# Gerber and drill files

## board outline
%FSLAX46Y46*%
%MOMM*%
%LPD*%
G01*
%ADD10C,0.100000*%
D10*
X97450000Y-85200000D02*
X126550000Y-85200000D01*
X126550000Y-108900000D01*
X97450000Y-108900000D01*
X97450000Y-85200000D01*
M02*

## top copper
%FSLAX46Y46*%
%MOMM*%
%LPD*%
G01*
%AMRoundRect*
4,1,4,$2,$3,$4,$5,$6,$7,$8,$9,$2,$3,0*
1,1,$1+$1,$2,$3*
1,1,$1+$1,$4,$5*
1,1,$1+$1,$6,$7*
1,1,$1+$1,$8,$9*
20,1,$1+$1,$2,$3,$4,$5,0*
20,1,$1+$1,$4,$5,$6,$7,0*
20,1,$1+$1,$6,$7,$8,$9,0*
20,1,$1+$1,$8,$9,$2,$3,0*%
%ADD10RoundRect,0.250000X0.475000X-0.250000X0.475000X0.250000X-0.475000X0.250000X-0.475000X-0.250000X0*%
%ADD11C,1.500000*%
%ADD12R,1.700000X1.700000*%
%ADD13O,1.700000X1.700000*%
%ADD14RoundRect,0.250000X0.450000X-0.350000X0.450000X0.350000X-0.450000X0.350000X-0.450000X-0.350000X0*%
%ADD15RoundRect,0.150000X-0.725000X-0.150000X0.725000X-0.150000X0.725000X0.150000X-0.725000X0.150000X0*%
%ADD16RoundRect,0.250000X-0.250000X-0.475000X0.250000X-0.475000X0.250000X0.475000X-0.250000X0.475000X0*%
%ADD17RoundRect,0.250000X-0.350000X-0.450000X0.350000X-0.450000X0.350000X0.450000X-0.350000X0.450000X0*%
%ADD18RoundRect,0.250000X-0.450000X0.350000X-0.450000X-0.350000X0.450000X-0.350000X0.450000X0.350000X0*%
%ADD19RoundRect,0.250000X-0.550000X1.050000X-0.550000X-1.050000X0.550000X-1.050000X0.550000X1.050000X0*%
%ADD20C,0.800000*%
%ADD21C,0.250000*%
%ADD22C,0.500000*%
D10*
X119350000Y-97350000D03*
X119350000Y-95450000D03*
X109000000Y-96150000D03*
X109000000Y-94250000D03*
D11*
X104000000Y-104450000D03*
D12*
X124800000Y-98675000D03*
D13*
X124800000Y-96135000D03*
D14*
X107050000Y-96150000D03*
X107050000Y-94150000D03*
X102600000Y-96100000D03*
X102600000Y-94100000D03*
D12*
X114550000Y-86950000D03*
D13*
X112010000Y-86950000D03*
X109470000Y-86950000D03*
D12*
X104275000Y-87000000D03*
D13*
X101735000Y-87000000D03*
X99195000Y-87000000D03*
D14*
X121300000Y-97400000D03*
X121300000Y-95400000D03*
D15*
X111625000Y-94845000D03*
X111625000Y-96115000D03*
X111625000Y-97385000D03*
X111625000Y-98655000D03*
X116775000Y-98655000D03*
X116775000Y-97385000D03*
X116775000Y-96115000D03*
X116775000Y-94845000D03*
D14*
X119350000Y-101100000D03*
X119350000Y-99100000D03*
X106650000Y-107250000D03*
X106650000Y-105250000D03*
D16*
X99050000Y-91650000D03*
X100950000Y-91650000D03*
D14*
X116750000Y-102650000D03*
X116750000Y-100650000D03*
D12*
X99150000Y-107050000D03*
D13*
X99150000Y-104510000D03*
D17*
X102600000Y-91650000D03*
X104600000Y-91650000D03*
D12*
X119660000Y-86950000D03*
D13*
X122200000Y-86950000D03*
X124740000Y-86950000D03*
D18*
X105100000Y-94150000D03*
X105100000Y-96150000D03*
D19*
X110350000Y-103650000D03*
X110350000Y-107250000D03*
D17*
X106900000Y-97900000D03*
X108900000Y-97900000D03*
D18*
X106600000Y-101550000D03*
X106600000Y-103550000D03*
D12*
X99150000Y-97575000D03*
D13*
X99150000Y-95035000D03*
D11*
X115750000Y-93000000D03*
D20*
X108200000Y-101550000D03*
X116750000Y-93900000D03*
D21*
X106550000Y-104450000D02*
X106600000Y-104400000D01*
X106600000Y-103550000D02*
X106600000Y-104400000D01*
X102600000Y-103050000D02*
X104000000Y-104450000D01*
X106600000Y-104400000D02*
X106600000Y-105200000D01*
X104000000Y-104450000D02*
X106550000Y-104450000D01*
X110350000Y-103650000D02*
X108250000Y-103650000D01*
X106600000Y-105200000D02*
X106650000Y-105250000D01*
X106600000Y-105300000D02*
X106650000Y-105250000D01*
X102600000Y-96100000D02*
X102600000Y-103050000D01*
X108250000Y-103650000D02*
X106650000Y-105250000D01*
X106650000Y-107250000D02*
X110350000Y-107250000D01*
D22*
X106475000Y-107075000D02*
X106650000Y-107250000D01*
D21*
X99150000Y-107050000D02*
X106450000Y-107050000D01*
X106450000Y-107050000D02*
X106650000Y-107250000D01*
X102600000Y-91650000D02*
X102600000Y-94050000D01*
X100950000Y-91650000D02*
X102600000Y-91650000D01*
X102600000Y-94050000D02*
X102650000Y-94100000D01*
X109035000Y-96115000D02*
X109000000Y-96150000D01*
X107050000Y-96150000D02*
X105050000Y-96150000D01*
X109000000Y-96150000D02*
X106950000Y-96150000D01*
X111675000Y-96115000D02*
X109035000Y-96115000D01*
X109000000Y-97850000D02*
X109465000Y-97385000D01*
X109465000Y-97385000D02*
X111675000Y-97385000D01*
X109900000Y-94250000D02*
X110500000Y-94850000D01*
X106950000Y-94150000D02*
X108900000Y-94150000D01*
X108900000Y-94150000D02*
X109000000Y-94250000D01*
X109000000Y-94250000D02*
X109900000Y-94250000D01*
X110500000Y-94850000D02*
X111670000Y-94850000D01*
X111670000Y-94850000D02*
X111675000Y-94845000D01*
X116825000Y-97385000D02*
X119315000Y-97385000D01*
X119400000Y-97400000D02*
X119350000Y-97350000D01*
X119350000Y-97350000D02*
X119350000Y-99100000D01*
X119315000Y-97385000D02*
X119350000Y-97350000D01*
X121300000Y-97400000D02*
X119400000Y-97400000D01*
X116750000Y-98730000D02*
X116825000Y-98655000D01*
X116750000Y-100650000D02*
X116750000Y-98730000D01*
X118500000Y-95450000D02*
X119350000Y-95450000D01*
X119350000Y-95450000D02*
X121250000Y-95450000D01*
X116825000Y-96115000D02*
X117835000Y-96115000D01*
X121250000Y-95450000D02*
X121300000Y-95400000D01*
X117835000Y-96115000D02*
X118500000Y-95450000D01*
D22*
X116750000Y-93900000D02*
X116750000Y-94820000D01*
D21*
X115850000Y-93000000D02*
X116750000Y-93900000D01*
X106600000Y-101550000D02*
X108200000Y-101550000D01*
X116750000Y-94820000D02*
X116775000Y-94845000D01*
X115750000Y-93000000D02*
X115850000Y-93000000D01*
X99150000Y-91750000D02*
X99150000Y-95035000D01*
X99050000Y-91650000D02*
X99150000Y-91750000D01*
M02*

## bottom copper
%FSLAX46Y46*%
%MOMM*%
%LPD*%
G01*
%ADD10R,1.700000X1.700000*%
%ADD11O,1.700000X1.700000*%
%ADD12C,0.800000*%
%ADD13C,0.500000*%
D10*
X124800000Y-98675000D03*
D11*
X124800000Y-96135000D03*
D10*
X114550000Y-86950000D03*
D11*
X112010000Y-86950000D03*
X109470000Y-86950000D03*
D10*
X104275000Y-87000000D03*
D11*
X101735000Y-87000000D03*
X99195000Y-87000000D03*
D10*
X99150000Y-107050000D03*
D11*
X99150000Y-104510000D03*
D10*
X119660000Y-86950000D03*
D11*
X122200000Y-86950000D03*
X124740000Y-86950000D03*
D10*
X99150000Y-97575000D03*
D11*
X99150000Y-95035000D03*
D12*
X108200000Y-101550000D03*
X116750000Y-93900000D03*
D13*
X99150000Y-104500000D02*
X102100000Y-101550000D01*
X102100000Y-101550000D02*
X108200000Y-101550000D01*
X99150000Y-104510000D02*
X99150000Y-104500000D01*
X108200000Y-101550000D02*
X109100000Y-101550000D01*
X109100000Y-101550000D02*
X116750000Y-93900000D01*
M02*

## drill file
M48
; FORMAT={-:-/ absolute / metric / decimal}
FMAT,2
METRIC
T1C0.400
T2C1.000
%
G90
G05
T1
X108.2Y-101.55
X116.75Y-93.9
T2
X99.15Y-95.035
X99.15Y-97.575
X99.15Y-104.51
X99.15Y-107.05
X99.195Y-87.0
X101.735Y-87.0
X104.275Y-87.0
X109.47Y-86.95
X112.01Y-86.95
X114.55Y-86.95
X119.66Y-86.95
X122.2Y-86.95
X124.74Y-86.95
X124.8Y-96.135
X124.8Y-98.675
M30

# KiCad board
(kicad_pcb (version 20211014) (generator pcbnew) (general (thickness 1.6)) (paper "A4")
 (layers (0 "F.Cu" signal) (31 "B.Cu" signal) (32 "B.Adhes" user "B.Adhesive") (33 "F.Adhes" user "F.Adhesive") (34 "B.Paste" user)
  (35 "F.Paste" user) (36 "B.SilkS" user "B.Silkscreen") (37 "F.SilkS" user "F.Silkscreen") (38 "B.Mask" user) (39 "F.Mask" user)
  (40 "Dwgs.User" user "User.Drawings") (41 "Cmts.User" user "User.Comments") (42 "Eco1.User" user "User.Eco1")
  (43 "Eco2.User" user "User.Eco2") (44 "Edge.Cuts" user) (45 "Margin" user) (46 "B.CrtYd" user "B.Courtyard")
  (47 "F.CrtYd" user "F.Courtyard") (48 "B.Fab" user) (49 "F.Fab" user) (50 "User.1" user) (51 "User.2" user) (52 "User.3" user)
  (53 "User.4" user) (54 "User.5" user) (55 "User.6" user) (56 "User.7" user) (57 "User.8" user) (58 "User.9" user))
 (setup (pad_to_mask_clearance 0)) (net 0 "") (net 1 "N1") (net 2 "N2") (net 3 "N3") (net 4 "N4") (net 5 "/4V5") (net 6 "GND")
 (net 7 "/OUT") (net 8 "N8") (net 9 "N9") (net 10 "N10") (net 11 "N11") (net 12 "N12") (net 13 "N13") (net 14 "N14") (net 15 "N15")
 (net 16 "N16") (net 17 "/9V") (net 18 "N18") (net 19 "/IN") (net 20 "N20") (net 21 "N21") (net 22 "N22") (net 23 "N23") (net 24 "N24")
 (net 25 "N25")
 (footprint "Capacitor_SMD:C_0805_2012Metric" (layer "F.Cu") (at 119.35 96.4 90)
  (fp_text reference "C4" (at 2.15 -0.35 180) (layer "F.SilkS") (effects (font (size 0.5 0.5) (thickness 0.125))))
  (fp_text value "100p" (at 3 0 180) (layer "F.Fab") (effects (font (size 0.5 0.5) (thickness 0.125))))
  (pad "1" smd roundrect (at -0.95 0 90) (size 1 1.45) (layers "F.Cu" "F.Paste" "F.Mask") (roundrect_rratio 0.25) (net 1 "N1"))
  (pad "2" smd roundrect (at 0.95 0 90) (size 1 1.45) (layers "F.Cu" "F.Paste" "F.Mask") (roundrect_rratio 0.25) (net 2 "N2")))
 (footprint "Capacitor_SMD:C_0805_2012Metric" (layer "F.Cu") (at 109 95.2 90)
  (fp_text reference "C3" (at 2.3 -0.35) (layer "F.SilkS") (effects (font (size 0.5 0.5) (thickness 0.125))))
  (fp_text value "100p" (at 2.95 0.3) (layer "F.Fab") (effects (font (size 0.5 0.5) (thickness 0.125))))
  (pad "1" smd roundrect (at -0.95 0 90) (size 1 1.45) (layers "F.Cu" "F.Paste" "F.Mask") (roundrect_rratio 0.25) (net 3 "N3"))
  (pad "2" smd roundrect (at 0.95 0 90) (size 1 1.45) (layers "F.Cu" "F.Paste" "F.Mask") (roundrect_rratio 0.25) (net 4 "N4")))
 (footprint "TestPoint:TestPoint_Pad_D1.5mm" (layer "F.Cu") (at 104 104.45)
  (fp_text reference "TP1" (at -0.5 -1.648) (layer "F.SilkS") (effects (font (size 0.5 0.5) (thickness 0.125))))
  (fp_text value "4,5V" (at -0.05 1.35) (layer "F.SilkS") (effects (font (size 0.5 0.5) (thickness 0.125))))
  (pad "1" smd circle (at 0 0) (size 1.5 1.5) (layers "F.Cu" "F.Mask") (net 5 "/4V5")))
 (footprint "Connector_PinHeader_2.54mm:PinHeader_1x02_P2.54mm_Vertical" (layer "F.Cu") (at 124.8 98.675 180)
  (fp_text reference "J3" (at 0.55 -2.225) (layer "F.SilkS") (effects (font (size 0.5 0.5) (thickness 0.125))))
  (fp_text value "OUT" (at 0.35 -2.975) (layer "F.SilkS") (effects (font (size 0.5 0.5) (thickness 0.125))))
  (pad "1" thru_hole rect (at 0 0 180) (size 1.7 1.7) (drill 1) (layers *.Cu *.Mask) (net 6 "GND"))
  (pad "2" thru_hole oval (at 0 2.54 180) (size 1.7 1.7) (drill 1) (layers *.Cu *.Mask) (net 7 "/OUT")))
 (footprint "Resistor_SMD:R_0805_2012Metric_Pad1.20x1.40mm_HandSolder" (layer "F.Cu") (at 107.05 95.15 90)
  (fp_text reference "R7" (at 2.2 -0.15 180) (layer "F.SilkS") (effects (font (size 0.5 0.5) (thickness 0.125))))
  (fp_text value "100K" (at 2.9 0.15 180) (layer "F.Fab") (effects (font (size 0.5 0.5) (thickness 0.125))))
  (pad "1" smd roundrect (at -1 0 90) (size 1.2 1.4) (layers "F.Cu" "F.Paste" "F.Mask") (roundrect_rratio 0.208333) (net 3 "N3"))
  (pad "2" smd roundrect (at 1 0 90) (size 1.2 1.4) (layers "F.Cu" "F.Paste" "F.Mask") (roundrect_rratio 0.208333) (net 4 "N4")))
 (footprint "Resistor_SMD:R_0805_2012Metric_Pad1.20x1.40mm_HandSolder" (layer "F.Cu") (at 102.6 95.1 90)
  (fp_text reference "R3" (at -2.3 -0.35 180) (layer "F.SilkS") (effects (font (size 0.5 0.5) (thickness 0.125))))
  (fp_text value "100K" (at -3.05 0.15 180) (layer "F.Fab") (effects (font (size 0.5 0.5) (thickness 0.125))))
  (pad "1" smd roundrect (at -1 0 90) (size 1.2 1.4) (layers "F.Cu" "F.Paste" "F.Mask") (roundrect_rratio 0.208333) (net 5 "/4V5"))
  (pad "2" smd roundrect (at 1 0 90) (size 1.2 1.4) (layers "F.Cu" "F.Paste" "F.Mask") (roundrect_rratio 0.208333) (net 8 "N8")))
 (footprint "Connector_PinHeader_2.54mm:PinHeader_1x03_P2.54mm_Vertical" (layer "F.Cu") (at 114.55 86.95 -90)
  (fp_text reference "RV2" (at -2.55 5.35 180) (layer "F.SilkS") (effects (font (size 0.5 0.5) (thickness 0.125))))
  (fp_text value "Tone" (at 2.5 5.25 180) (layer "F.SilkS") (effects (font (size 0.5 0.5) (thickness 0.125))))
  (pad "1" thru_hole rect (at 0 0 270) (size 1.7 1.7) (drill 1) (layers *.Cu *.Mask) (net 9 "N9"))
  (pad "2" thru_hole oval (at 0 2.54 270) (size 1.7 1.7) (drill 1) (layers *.Cu *.Mask) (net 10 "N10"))
  (pad "3" thru_hole oval (at 0 5.08 270) (size 1.7 1.7) (drill 1) (layers *.Cu *.Mask) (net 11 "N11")))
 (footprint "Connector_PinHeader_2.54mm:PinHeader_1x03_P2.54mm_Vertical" (layer "F.Cu") (at 104.275 87 -90)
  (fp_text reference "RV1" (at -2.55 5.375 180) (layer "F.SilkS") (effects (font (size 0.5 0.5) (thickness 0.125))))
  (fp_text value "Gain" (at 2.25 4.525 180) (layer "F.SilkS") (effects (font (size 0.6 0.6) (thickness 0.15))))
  (pad "1" thru_hole rect (at 0 0 270) (size 1.7 1.7) (drill 1) (layers *.Cu *.Mask) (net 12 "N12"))
  (pad "2" thru_hole oval (at 0 2.54 270) (size 1.7 1.7) (drill 1) (layers *.Cu *.Mask) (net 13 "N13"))
  (pad "3" thru_hole oval (at 0 5.08 270) (size 1.7 1.7) (drill 1) (layers *.Cu *.Mask) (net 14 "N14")))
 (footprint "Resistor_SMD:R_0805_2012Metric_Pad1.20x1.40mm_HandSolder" (layer "F.Cu") (at 121.3 96.4 90)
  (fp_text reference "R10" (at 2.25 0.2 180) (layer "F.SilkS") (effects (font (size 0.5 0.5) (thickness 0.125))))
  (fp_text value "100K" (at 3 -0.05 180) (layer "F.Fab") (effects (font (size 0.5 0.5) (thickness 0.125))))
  (pad "1" smd roundrect (at -1 0 90) (size 1.2 1.4) (layers "F.Cu" "F.Paste" "F.Mask") (roundrect_rratio 0.208333) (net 1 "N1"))
  (pad "2" smd roundrect (at 1 0 90) (size 1.2 1.4) (layers "F.Cu" "F.Paste" "F.Mask") (roundrect_rratio 0.208333) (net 2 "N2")))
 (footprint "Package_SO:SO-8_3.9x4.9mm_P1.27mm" (layer "F.Cu") (at 114.2 96.75)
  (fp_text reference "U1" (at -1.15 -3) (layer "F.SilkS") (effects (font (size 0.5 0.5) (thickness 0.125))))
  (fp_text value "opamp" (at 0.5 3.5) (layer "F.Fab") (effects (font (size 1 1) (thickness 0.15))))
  (pad "1" smd roundrect (at -2.575 -1.905) (size 1.75 0.6) (layers "F.Cu" "F.Paste" "F.Mask") (roundrect_rratio 0.25) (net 4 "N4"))
  (pad "2" smd roundrect (at -2.575 -0.635) (size 1.75 0.6) (layers "F.Cu" "F.Paste" "F.Mask") (roundrect_rratio 0.25) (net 3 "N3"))
  (pad "3" smd roundrect (at -2.575 0.635) (size 1.75 0.6) (layers "F.Cu" "F.Paste" "F.Mask") (roundrect_rratio 0.25) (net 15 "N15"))
  (pad "4" smd roundrect (at -2.575 1.905) (size 1.75 0.6) (layers "F.Cu" "F.Paste" "F.Mask") (roundrect_rratio 0.25) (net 6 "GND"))
  (pad "5" smd roundrect (at 2.575 1.905) (size 1.75 0.6) (layers "F.Cu" "F.Paste" "F.Mask") (roundrect_rratio 0.25) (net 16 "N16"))
  (pad "6" smd roundrect (at 2.575 0.635) (size 1.75 0.6) (layers "F.Cu" "F.Paste" "F.Mask") (roundrect_rratio 0.25) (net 1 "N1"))
  (pad "7" smd roundrect (at 2.575 -0.635) (size 1.75 0.6) (layers "F.Cu" "F.Paste" "F.Mask") (roundrect_rratio 0.25) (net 2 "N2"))
  (pad "8" smd roundrect (at 2.575 -1.905) (size 1.75 0.6) (layers "F.Cu" "F.Paste" "F.Mask") (roundrect_rratio 0.25) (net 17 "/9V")))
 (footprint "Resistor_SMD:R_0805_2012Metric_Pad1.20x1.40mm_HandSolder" (layer "F.Cu") (at 119.35 100.1 90)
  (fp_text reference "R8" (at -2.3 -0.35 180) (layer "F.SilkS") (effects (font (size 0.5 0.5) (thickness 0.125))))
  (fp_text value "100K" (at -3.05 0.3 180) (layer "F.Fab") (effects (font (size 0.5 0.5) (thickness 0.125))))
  (pad "1" smd roundrect (at -1 0 90) (size 1.2 1.4) (layers "F.Cu" "F.Paste" "F.Mask") (roundrect_rratio 0.208333) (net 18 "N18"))
  (pad "2" smd roundrect (at 1 0 90) (size 1.2 1.4) (layers "F.Cu" "F.Paste" "F.Mask") (roundrect_rratio 0.208333) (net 1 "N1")))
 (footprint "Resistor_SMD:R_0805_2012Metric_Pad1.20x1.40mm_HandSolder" (layer "F.Cu") (at 106.65 106.25 90)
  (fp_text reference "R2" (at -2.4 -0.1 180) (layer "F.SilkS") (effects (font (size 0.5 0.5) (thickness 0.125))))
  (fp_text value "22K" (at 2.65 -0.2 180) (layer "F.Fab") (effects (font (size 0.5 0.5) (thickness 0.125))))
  (pad "1" smd roundrect (at -1 0 90) (size 1.2 1.4) (layers "F.Cu" "F.Paste" "F.Mask") (roundrect_rratio 0.208333) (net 6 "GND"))
  (pad "2" smd roundrect (at 1 0 90) (size 1.2 1.4) (layers "F.Cu" "F.Paste" "F.Mask") (roundrect_rratio 0.208333) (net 5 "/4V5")))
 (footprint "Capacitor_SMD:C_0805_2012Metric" (layer "F.Cu") (at 100 91.65)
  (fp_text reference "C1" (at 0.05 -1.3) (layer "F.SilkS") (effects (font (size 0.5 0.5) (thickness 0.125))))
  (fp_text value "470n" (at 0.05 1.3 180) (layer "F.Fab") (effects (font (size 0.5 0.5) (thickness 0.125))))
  (pad "1" smd roundrect (at -0.95 0) (size 1 1.45) (layers "F.Cu" "F.Paste" "F.Mask") (roundrect_rratio 0.25) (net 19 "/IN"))
  (pad "2" smd roundrect (at 0.95 0) (size 1 1.45) (layers "F.Cu" "F.Paste" "F.Mask") (roundrect_rratio 0.25) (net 8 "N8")))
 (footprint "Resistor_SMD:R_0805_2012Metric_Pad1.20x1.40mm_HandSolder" (layer "F.Cu") (at 116.75 101.65 90)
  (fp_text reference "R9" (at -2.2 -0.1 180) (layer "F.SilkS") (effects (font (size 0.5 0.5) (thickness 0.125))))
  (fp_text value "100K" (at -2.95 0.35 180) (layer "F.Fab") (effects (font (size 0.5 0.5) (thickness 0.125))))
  (pad "1" smd roundrect (at -1 0 90) (size 1.2 1.4) (layers "F.Cu" "F.Paste" "F.Mask") (roundrect_rratio 0.208333) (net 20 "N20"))
  (pad "2" smd roundrect (at 1 0 90) (size 1.2 1.4) (layers "F.Cu" "F.Paste" "F.Mask") (roundrect_rratio 0.208333) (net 16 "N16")))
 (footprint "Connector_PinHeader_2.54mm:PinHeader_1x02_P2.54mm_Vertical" (layer "F.Cu") (at 99.15 107.05 180)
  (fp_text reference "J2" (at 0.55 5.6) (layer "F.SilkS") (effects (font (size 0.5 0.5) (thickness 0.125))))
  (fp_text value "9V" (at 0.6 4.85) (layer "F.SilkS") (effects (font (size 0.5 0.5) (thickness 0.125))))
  (pad "1" thru_hole rect (at 0 0 180) (size 1.7 1.7) (drill 1) (layers *.Cu *.Mask) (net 6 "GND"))
  (pad "2" thru_hole oval (at 0 2.54 180) (size 1.7 1.7) (drill 1) (layers *.Cu *.Mask) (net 17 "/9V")))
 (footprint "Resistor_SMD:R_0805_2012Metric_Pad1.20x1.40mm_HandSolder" (layer "F.Cu") (at 103.6 91.65)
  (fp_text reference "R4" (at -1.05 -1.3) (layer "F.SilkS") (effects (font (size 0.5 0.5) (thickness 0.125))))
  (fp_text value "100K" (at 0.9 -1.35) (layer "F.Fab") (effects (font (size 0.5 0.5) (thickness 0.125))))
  (pad "1" smd roundrect (at -1 0) (size 1.2 1.4) (layers "F.Cu" "F.Paste" "F.Mask") (roundrect_rratio 0.208333) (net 8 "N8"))
  (pad "2" smd roundrect (at 1 0) (size 1.2 1.4) (layers "F.Cu" "F.Paste" "F.Mask") (roundrect_rratio 0.208333) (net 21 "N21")))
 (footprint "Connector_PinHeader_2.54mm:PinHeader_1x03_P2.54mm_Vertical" (layer "F.Cu") (at 119.66 86.95 90)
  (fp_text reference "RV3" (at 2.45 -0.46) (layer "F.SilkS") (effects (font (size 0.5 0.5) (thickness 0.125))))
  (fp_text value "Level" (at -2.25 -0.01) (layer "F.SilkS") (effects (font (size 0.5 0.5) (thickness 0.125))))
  (pad "1" thru_hole rect (at 0 0 90) (size 1.7 1.7) (drill 1) (layers *.Cu *.Mask) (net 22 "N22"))
  (pad "2" thru_hole oval (at 0 2.54 90) (size 1.7 1.7) (drill 1) (layers *.Cu *.Mask) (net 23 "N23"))
  (pad "3" thru_hole oval (at 0 5.08 90) (size 1.7 1.7) (drill 1) (layers *.Cu *.Mask) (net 6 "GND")))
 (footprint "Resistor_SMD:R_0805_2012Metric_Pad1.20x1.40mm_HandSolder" (layer "F.Cu") (at 105.1 95.15 -90)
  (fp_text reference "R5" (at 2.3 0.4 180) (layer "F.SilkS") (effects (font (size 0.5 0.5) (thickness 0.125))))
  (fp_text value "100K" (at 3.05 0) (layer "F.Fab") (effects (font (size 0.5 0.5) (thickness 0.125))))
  (pad "1" smd roundrect (at -1 0 270) (size 1.2 1.4) (layers "F.Cu" "F.Paste" "F.Mask") (roundrect_rratio 0.208333) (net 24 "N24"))
  (pad "2" smd roundrect (at 1 0 270) (size 1.2 1.4) (layers "F.Cu" "F.Paste" "F.Mask") (roundrect_rratio 0.208333) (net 3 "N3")))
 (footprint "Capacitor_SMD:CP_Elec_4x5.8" (layer "F.Cu") (at 110.35 105.45 -90)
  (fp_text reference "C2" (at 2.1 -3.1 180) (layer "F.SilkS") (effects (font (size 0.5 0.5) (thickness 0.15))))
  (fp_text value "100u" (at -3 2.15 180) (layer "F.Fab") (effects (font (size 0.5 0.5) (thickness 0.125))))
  (pad "1" smd roundrect (at -1.8 0 270) (size 2.6 1.6) (layers "F.Cu" "F.Paste" "F.Mask") (roundrect_rratio 0.15625) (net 5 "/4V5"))
  (pad "2" smd roundrect (at 1.8 0 270) (size 2.6 1.6) (layers "F.Cu" "F.Paste" "F.Mask") (roundrect_rratio 0.15625) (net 6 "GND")))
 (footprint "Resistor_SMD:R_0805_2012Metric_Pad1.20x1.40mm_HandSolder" (layer "F.Cu") (at 107.9 97.9)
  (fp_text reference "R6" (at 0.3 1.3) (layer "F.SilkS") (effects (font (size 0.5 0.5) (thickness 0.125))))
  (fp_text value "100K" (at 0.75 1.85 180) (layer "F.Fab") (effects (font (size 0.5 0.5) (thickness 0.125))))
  (pad "1" smd roundrect (at -1 0) (size 1.2 1.4) (layers "F.Cu" "F.Paste" "F.Mask") (roundrect_rratio 0.208333) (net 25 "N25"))
  (pad "2" smd roundrect (at 1 0) (size 1.2 1.4) (layers "F.Cu" "F.Paste" "F.Mask") (roundrect_rratio 0.208333) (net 15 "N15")))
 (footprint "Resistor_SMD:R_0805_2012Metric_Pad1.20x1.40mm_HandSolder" (layer "F.Cu") (at 106.6 102.55 -90)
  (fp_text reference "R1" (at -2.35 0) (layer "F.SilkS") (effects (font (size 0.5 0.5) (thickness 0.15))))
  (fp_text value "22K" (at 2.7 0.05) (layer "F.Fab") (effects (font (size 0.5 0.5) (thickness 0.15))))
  (pad "1" smd roundrect (at -1 0 270) (size 1.2 1.4) (layers "F.Cu" "F.Paste" "F.Mask") (roundrect_rratio 0.208333) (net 17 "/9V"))
  (pad "2" smd roundrect (at 1 0 270) (size 1.2 1.4) (layers "F.Cu" "F.Paste" "F.Mask") (roundrect_rratio 0.208333) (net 5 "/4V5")))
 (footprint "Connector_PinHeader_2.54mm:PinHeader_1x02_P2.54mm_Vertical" (layer "F.Cu") (at 99.15 97.575 180)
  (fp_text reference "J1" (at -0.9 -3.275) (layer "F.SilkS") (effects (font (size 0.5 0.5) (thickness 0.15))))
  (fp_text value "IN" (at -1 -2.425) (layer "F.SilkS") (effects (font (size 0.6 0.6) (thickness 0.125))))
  (pad "1" thru_hole rect (at 0 0 180) (size 1.7 1.7) (drill 1) (layers *.Cu *.Mask) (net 6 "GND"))
  (pad "2" thru_hole oval (at 0 2.54 180) (size 1.7 1.7) (drill 1) (layers *.Cu *.Mask) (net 19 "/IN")))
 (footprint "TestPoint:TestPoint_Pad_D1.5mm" (layer "F.Cu") (at 115.75 93)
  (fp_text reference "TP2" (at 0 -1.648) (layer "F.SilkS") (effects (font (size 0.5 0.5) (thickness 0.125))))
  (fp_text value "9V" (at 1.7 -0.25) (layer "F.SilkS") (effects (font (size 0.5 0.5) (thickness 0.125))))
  (pad "1" smd circle (at 0 0) (size 1.5 1.5) (layers "F.Cu" "F.Mask") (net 17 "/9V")))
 (gr_rect (start 97.45 85.2) (end 126.55 108.9) (layer "Edge.Cuts") (width 0.1) (fill none))
 (segment (start 106.55 104.45) (end 106.6 104.4) (width 0.25) (layer "F.Cu") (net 5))
 (segment (start 106.6 103.55) (end 106.6 104.4) (width 0.25) (layer "F.Cu") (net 5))
 (segment (start 102.6 103.05) (end 104 104.45) (width 0.25) (layer "F.Cu") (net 5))
 (segment (start 106.6 104.4) (end 106.6 105.2) (width 0.25) (layer "F.Cu") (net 5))
 (segment (start 104 104.45) (end 106.55 104.45) (width 0.25) (layer "F.Cu") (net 5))
 (segment (start 110.35 103.65) (end 108.25 103.65) (width 0.25) (layer "F.Cu") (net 5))
 (segment (start 106.6 105.2) (end 106.65 105.25) (width 0.25) (layer "F.Cu") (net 5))
 (segment (start 106.6 105.3) (end 106.65 105.25) (width 0.25) (layer "F.Cu") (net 5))
 (segment (start 102.6 96.1) (end 102.6 103.05) (width 0.25) (layer "F.Cu") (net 5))
 (segment (start 108.25 103.65) (end 106.65 105.25) (width 0.25) (layer "F.Cu") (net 5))
 (segment (start 106.65 107.25) (end 110.35 107.25) (width 0.25) (layer "F.Cu") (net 6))
 (segment (start 106.475 107.075) (end 106.65 107.25) (width 0.5) (layer "F.Cu") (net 6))
 (segment (start 99.15 107.05) (end 106.45 107.05) (width 0.25) (layer "F.Cu") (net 6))
 (segment (start 106.45 107.05) (end 106.65 107.25) (width 0.25) (layer "F.Cu") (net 6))
 (segment (start 102.6 91.65) (end 102.6 94.05) (width 0.25) (layer "F.Cu") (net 8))
 (segment (start 100.95 91.65) (end 102.6 91.65) (width 0.25) (layer "F.Cu") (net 8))
 (segment (start 102.6 94.05) (end 102.65 94.1) (width 0.25) (layer "F.Cu") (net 8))
 (segment (start 109.035 96.115) (end 109 96.15) (width 0.25) (layer "F.Cu") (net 3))
 (segment (start 107.05 96.15) (end 105.05 96.15) (width 0.25) (layer "F.Cu") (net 3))
 (segment (start 109 96.15) (end 106.95 96.15) (width 0.25) (layer "F.Cu") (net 3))
 (segment (start 111.675 96.115) (end 109.035 96.115) (width 0.25) (layer "F.Cu") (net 3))
 (segment (start 109 97.85) (end 109.465 97.385) (width 0.25) (layer "F.Cu") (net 15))
 (segment (start 109.465 97.385) (end 111.675 97.385) (width 0.25) (layer "F.Cu") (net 15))
 (segment (start 109.9 94.25) (end 110.5 94.85) (width 0.25) (layer "F.Cu") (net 4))
 (segment (start 106.95 94.15) (end 108.9 94.15) (width 0.25) (layer "F.Cu") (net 4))
 (segment (start 108.9 94.15) (end 109 94.25) (width 0.25) (layer "F.Cu") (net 4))
 (segment (start 109 94.25) (end 109.9 94.25) (width 0.25) (layer "F.Cu") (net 4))
 (segment (start 110.5 94.85) (end 111.67 94.85) (width 0.25) (layer "F.Cu") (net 4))
 (segment (start 111.67 94.85) (end 111.675 94.845) (width 0.25) (layer "F.Cu") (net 4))
 (segment (start 116.825 97.385) (end 119.315 97.385) (width 0.25) (layer "F.Cu") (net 1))
 (segment (start 119.4 97.4) (end 119.35 97.35) (width 0.25) (layer "F.Cu") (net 1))
 (segment (start 119.35 97.35) (end 119.35 99.1) (width 0.25) (layer "F.Cu") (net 1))
 (segment (start 119.315 97.385) (end 119.35 97.35) (width 0.25) (layer "F.Cu") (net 1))
 (segment (start 121.3 97.4) (end 119.4 97.4) (width 0.25) (layer "F.Cu") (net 1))
 (segment (start 116.75 98.73) (end 116.825 98.655) (width 0.25) (layer "F.Cu") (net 16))
 (segment (start 116.75 100.65) (end 116.75 98.73) (width 0.25) (layer "F.Cu") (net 16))
 (segment (start 118.5 95.45) (end 119.35 95.45) (width 0.25) (layer "F.Cu") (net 2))
 (segment (start 119.35 95.45) (end 121.25 95.45) (width 0.25) (layer "F.Cu") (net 2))
 (segment (start 116.825 96.115) (end 117.835 96.115) (width 0.25) (layer "F.Cu") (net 2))
 (segment (start 121.25 95.45) (end 121.3 95.4) (width 0.25) (layer "F.Cu") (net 2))
 (segment (start 117.835 96.115) (end 118.5 95.45) (width 0.25) (layer "F.Cu") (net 2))
 (segment (start 116.75 93.9) (end 116.75 94.82) (width 0.5) (layer "F.Cu") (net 17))
 (segment (start 115.85 93) (end 116.75 93.9) (width 0.25) (layer "F.Cu") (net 17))
 (segment (start 106.6 101.55) (end 108.2 101.55) (width 0.25) (layer "F.Cu") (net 17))
 (segment (start 116.75 94.82) (end 116.775 94.845) (width 0.25) (layer "F.Cu") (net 17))
 (segment (start 115.75 93) (end 115.85 93) (width 0.25) (layer "F.Cu") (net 17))
 (via (at 108.2 101.55) (size 0.8) (drill 0.4) (layers "F.Cu" "B.Cu") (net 17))
 (via (at 116.75 93.9) (size 0.8) (drill 0.4) (layers "F.Cu" "B.Cu") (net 17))
 (segment (start 99.15 104.5) (end 102.1 101.55) (width 0.5) (layer "B.Cu") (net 17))
 (segment (start 102.1 101.55) (end 108.2 101.55) (width 0.5) (layer "B.Cu") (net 17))
 (segment (start 99.15 104.51) (end 99.15 104.5) (width 0.5) (layer "B.Cu") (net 17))
 (segment (start 108.2 101.55) (end 109.1 101.55) (width 0.5) (layer "B.Cu") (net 17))
 (segment (start 109.1 101.55) (end 116.75 93.9) (width 0.5) (layer "B.Cu") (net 17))
 (segment (start 99.15 91.75) (end 99.15 95.035) (width 0.25) (layer "F.Cu") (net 19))
 (segment (start 99.05 91.65) (end 99.15 91.75) (width 0.25) (layer "F.Cu") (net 19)))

